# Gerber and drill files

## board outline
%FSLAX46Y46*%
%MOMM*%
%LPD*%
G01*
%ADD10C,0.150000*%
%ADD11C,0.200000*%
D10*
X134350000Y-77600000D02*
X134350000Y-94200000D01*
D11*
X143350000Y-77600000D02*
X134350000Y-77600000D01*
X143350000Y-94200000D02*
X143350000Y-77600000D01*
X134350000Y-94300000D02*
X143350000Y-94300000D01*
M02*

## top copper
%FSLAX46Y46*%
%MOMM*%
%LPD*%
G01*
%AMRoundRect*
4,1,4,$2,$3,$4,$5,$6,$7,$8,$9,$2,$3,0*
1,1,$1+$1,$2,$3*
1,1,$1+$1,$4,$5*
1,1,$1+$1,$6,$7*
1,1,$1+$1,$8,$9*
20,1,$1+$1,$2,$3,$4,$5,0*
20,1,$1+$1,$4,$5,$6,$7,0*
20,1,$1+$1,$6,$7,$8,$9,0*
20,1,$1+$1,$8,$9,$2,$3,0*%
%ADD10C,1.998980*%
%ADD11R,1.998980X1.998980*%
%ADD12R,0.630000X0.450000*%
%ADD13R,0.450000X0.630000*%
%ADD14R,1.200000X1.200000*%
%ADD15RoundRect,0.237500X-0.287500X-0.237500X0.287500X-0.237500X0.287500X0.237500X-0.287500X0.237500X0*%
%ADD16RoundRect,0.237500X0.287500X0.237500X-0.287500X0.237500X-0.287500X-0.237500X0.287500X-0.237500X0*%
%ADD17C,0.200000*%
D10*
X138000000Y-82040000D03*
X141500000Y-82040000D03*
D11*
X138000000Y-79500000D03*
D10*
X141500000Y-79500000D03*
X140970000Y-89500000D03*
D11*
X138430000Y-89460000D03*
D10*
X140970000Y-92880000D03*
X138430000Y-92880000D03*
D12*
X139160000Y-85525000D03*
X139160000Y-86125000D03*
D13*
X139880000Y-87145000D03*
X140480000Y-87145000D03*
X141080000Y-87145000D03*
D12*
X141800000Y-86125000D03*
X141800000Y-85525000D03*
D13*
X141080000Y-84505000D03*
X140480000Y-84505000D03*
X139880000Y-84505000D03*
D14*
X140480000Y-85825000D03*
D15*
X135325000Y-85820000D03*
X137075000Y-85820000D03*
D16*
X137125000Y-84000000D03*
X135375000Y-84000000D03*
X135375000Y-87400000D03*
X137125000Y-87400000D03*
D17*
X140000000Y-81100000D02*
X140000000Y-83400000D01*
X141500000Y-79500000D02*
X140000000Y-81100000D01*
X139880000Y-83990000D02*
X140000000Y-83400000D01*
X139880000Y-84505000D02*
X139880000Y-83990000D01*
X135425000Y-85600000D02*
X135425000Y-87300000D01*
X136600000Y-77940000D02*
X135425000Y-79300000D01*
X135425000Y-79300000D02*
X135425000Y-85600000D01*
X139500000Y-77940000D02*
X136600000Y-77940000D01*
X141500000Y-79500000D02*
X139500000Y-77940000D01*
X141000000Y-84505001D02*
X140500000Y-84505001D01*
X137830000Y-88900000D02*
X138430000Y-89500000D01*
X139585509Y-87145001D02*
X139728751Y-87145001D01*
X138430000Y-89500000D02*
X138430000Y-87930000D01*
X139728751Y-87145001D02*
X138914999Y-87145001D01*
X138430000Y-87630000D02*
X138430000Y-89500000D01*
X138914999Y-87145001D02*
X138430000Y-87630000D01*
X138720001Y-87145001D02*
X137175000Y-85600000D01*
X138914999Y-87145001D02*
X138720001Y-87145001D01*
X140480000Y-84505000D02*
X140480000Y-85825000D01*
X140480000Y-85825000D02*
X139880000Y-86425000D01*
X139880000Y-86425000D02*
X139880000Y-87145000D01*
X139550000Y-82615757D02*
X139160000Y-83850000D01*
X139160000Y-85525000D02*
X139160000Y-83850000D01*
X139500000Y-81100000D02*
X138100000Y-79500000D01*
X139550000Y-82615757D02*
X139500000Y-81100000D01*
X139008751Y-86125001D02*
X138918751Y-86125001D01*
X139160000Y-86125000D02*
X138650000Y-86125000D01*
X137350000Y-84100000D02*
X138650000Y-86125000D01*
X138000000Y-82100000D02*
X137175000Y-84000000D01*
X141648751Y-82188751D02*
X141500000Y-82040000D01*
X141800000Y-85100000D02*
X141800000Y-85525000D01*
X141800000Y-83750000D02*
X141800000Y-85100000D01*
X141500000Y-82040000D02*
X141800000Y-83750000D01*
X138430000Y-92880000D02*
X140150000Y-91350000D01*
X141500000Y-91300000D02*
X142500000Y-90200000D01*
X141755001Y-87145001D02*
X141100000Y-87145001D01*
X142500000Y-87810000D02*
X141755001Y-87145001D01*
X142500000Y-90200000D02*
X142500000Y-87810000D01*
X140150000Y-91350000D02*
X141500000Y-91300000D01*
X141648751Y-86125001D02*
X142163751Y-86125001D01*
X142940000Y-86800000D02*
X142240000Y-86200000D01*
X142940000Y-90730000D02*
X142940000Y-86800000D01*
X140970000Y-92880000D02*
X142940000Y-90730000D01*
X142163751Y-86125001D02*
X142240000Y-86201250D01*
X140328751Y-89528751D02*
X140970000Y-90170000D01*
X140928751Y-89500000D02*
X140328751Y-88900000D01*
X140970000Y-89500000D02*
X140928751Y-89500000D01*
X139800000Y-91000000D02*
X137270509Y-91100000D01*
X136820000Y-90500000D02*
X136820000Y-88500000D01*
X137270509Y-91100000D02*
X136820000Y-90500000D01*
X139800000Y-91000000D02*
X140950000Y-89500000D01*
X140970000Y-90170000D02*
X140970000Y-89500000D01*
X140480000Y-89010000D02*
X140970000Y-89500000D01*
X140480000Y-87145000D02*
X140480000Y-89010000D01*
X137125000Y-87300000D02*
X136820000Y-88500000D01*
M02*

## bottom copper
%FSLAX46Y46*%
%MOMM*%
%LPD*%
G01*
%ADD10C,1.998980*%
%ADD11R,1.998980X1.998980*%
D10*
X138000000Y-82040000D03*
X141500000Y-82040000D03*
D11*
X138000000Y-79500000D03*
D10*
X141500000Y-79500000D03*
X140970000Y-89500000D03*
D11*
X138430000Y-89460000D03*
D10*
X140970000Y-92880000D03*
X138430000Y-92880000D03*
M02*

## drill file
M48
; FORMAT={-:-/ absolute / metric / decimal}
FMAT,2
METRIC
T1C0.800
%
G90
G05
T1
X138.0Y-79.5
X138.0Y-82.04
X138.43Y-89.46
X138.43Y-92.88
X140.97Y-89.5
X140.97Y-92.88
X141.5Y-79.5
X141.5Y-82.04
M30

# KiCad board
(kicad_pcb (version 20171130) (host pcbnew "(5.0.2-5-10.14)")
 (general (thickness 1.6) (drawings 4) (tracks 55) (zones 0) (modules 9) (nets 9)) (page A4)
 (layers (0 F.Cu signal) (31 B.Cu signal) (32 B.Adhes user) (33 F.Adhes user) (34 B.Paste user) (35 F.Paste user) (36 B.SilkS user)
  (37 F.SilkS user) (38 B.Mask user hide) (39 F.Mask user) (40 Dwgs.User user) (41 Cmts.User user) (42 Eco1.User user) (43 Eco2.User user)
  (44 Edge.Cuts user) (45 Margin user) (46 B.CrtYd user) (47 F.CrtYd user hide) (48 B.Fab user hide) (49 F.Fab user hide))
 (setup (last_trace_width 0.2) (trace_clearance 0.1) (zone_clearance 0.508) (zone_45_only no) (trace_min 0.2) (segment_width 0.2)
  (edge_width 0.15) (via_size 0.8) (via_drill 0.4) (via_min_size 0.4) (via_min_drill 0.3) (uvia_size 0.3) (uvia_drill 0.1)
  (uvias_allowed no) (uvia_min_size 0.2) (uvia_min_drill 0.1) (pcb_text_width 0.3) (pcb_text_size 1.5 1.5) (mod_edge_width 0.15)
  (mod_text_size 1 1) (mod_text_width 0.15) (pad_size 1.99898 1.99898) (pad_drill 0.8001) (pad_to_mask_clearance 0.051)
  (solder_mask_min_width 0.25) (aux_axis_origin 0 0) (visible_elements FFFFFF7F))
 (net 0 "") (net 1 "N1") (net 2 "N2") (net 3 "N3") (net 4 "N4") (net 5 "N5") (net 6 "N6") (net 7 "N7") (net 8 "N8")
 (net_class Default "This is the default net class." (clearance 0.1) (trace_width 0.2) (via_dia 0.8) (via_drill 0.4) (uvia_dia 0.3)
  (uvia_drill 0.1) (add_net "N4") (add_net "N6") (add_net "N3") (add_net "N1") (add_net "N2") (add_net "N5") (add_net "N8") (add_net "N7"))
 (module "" (layer F.Cu) (at 140.97 77.47)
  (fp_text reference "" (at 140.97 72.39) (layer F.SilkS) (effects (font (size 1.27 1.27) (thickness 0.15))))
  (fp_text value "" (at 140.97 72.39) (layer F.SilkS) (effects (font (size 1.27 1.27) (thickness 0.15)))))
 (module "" (layer F.Cu) (at 140.97 77.47)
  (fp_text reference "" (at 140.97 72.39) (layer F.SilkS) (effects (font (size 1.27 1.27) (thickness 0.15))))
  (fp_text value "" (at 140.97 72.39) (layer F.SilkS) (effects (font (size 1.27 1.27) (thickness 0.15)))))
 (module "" (layer F.Cu) (at 140.97 72.39)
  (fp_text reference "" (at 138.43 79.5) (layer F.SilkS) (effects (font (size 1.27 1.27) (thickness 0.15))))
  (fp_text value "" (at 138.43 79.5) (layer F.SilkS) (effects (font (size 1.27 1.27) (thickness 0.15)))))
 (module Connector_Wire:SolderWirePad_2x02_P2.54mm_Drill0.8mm (layer F.Cu) (at 138.43 79.5)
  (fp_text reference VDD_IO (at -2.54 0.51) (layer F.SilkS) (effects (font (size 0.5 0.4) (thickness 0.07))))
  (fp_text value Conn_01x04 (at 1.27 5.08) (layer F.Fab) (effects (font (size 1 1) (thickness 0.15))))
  (pad 3 thru_hole circle (at -0.43 2.54) (size 1.99898 1.99898) (drill 0.8001) (layers *.Cu *.Mask) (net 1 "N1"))
  (pad 4 thru_hole circle (at 3.07 2.54) (size 1.99898 1.99898) (drill 0.8001) (layers *.Cu *.Mask) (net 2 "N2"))
  (pad 1 thru_hole rect (at -0.43 0) (size 1.99898 1.99898) (drill 0.8001) (layers *.Cu *.Mask) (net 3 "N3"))
  (pad 2 thru_hole circle (at 3.07 0) (size 1.99898 1.99898) (drill 0.8001) (layers *.Cu *.Mask) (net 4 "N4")))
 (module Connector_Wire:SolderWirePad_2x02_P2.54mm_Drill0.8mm (layer F.Cu) (at 138.43 89.5)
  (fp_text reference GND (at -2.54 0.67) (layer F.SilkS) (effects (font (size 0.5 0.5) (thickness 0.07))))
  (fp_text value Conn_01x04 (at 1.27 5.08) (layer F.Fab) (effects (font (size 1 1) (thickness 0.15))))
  (pad 2 thru_hole circle (at 2.54 0) (size 1.99898 1.99898) (drill 0.8001) (layers *.Cu *.Mask) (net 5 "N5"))
  (pad 1 thru_hole rect (at 0 -0.04) (size 1.99898 1.99898) (drill 0.8001) (layers *.Cu *.Mask) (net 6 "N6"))
  (pad 4 thru_hole circle (at 2.54 3.38) (size 1.99898 1.99898) (drill 0.8001) (layers *.Cu *.Mask) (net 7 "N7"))
  (pad 3 thru_hole circle (at 0 3.38) (size 1.99898 1.99898) (drill 0.8001) (layers *.Cu *.Mask) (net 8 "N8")))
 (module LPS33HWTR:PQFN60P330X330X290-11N (layer F.Cu) (at 140.48 85.825)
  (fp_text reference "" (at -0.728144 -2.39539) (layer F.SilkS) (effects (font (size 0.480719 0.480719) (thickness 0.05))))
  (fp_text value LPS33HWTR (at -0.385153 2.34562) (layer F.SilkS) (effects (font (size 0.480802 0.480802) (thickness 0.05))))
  (pad 1 smd rect (at -1.32 -0.3) (size 0.63 0.45) (layers F.Cu F.Paste F.Mask) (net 3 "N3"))
  (pad 2 smd rect (at -1.32 0.3) (size 0.63 0.45) (layers F.Cu F.Paste F.Mask) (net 1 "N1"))
  (pad 3 smd rect (at -0.6 1.32 90) (size 0.63 0.45) (layers F.Cu F.Paste F.Mask) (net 6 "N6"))
  (pad 4 smd rect (at 0 1.32 90) (size 0.63 0.45) (layers F.Cu F.Paste F.Mask) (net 5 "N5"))
  (pad 5 smd rect (at 0.6 1.32 90) (size 0.63 0.45) (layers F.Cu F.Paste F.Mask) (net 8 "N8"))
  (pad 6 smd rect (at 1.32 0.3 180) (size 0.63 0.45) (layers F.Cu F.Paste F.Mask) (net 7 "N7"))
  (pad 7 smd rect (at 1.32 -0.3 180) (size 0.63 0.45) (layers F.Cu F.Paste F.Mask) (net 2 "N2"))
  (pad 8 smd rect (at 0.6 -1.32 270) (size 0.63 0.45) (layers F.Cu F.Paste F.Mask) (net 6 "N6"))
  (pad 9 smd rect (at 0 -1.32 270) (size 0.63 0.45) (layers F.Cu F.Paste F.Mask) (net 6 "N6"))
  (pad 10 smd rect (at -0.6 -1.32 270) (size 0.63 0.45) (layers F.Cu F.Paste F.Mask) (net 4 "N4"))
  (pad EP smd rect (at 0 0) (size 1.2 1.2) (layers F.Cu F.Paste F.Mask) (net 6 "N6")))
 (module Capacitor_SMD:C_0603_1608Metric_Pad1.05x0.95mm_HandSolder (layer F.Cu) (at 136.2 85.82)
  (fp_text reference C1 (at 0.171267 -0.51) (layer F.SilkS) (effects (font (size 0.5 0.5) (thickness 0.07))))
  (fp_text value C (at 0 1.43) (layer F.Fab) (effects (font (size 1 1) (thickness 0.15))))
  (pad 1 smd roundrect (at -0.875 0) (size 1.05 0.95) (layers F.Cu F.Paste F.Mask) (roundrect_rratio 0.25) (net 4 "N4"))
  (pad 2 smd roundrect (at 0.875 0) (size 1.05 0.95) (layers F.Cu F.Paste F.Mask) (roundrect_rratio 0.25) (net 6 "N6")))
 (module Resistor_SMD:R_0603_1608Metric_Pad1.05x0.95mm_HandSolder (layer F.Cu) (at 136.25 84 180)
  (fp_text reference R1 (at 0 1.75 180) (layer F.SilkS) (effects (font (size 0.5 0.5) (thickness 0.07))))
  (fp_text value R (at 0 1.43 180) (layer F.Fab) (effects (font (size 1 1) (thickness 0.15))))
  (pad 1 smd roundrect (at -0.875 0 180) (size 1.05 0.95) (layers F.Cu F.Paste F.Mask) (roundrect_rratio 0.25) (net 1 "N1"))
  (pad 2 smd roundrect (at 0.875 0 180) (size 1.05 0.95) (layers F.Cu F.Paste F.Mask) (roundrect_rratio 0.25) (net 4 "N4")))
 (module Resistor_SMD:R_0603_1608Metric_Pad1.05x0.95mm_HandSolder (layer F.Cu) (at 136.25 87.4 180)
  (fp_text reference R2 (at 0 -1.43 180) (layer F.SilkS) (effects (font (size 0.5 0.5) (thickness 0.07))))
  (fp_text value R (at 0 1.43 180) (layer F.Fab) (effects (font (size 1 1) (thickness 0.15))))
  (pad 2 smd roundrect (at 0.875 0 180) (size 1.05 0.95) (layers F.Cu F.Paste F.Mask) (roundrect_rratio 0.25) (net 4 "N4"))
  (pad 1 smd roundrect (at -0.875 0 180) (size 1.05 0.95) (layers F.Cu F.Paste F.Mask) (roundrect_rratio 0.25) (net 5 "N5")))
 (gr_line (start 134.35 77.6) (end 134.35 94.2) (layer Edge.Cuts) (width 0.15))
 (gr_line (start 143.35 77.6) (end 134.35 77.6) (layer Edge.Cuts) (width 0.2))
 (gr_line (start 143.35 94.2) (end 143.35 77.6) (layer Edge.Cuts) (width 0.2))
 (gr_line (start 134.35 94.3) (end 143.35 94.3) (layer Edge.Cuts) (width 0.2))
 (segment (start 140 81.1) (end 140 83.4) (width 0.2) (layer F.Cu) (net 4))
 (segment (start 141.5 79.5) (end 140 81.1) (width 0.2) (layer F.Cu) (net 4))
 (segment (start 139.88 83.99) (end 140 83.4) (width 0.2) (layer F.Cu) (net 4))
 (segment (start 139.88 84.505) (end 139.88 83.99) (width 0.2) (layer F.Cu) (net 4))
 (segment (start 135.425 85.6) (end 135.425 87.3) (width 0.2) (layer F.Cu) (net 4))
 (segment (start 136.6 77.94) (end 135.425 79.3) (width 0.2) (layer F.Cu) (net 4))
 (segment (start 135.425 79.3) (end 135.425 85.6) (width 0.2) (layer F.Cu) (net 4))
 (segment (start 139.5 77.94) (end 136.6 77.94) (width 0.2) (layer F.Cu) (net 4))
 (segment (start 141.5 79.5) (end 139.5 77.94) (width 0.2) (layer F.Cu) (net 4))
 (segment (start 141 84.505001) (end 140.5 84.505001) (width 0.2) (layer F.Cu) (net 6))
 (segment (start 137.83 88.9) (end 138.43 89.5) (width 0.2) (layer F.Cu) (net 6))
 (segment (start 139.585509 87.145001) (end 139.728751 87.145001) (width 0.2) (layer F.Cu) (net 6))
 (segment (start 138.43 89.5) (end 138.43 87.93) (width 0.2) (layer F.Cu) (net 6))
 (segment (start 139.728751 87.145001) (end 138.914999 87.145001) (width 0.2) (layer F.Cu) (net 6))
 (segment (start 138.43 87.63) (end 138.43 89.5) (width 0.2) (layer F.Cu) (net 6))
 (segment (start 138.914999 87.145001) (end 138.43 87.63) (width 0.2) (layer F.Cu) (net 6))
 (segment (start 138.720001 87.145001) (end 137.175 85.6) (width 0.2) (layer F.Cu) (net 6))
 (segment (start 138.914999 87.145001) (end 138.720001 87.145001) (width 0.2) (layer F.Cu) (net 6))
 (segment (start 140.48 84.505) (end 140.48 85.825) (width 0.2) (layer F.Cu) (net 6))
 (segment (start 140.48 85.825) (end 139.88 86.425) (width 0.2) (layer F.Cu) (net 6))
 (segment (start 139.88 86.425) (end 139.88 87.145) (width 0.2) (layer F.Cu) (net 6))
 (segment (start 139.55 82.615757) (end 139.16 83.85) (width 0.2) (layer F.Cu) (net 3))
 (segment (start 139.16 85.525) (end 139.16 83.85) (width 0.2) (layer F.Cu) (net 3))
 (segment (start 139.5 81.1) (end 138.1 79.5) (width 0.2) (layer F.Cu) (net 3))
 (segment (start 139.55 82.615757) (end 139.5 81.1) (width 0.2) (layer F.Cu) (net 3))
 (segment (start 139.008751 86.125001) (end 138.918751 86.125001) (width 0.2) (layer F.Cu) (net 1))
 (segment (start 139.16 86.125) (end 138.65 86.125) (width 0.2) (layer F.Cu) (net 1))
 (segment (start 137.35 84.1) (end 138.65 86.125) (width 0.2) (layer F.Cu) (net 1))
 (segment (start 138 82.1) (end 137.175 84) (width 0.2) (layer F.Cu) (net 1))
 (segment (start 141.648751 82.188751) (end 141.5 82.04) (width 0.2) (layer F.Cu) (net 2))
 (segment (start 141.8 85.1) (end 141.8 85.525) (width 0.2) (layer F.Cu) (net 2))
 (segment (start 141.8 83.75) (end 141.8 85.1) (width 0.2) (layer F.Cu) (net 2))
 (segment (start 141.5 82.04) (end 141.8 83.75) (width 0.2) (layer F.Cu) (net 2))
 (segment (start 138.43 92.88) (end 140.15 91.35) (width 0.2) (layer F.Cu) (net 8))
 (segment (start 141.5 91.3) (end 142.5 90.2) (width 0.2) (layer F.Cu) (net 8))
 (segment (start 141.755001 87.145001) (end 141.1 87.145001) (width 0.2) (layer F.Cu) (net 8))
 (segment (start 142.5 87.81) (end 141.755001 87.145001) (width 0.2) (layer F.Cu) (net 8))
 (segment (start 142.5 90.2) (end 142.5 87.81) (width 0.2) (layer F.Cu) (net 8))
 (segment (start 140.15 91.35) (end 141.5 91.3) (width 0.2) (layer F.Cu) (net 8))
 (segment (start 141.648751 86.125001) (end 142.163751 86.125001) (width 0.2) (layer F.Cu) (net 7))
 (segment (start 142.94 86.8) (end 142.24 86.2) (width 0.2) (layer F.Cu) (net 7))
 (segment (start 142.94 90.73) (end 142.94 86.8) (width 0.2) (layer F.Cu) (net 7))
 (segment (start 140.97 92.88) (end 142.94 90.73) (width 0.2) (layer F.Cu) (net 7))
 (segment (start 142.163751 86.125001) (end 142.24 86.20125) (width 0.2) (layer F.Cu) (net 7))
 (segment (start 140.328751 89.528751) (end 140.97 90.17) (width 0.2) (layer F.Cu) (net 5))
 (segment (start 140.928751 89.5) (end 140.328751 88.9) (width 0.2) (layer F.Cu) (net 5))
 (segment (start 140.97 89.5) (end 140.928751 89.5) (width 0.2) (layer F.Cu) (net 5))
 (segment (start 139.8 91) (end 137.270509 91.1) (width 0.2) (layer F.Cu) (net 5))
 (segment (start 136.82 90.5) (end 136.82 88.5) (width 0.2) (layer F.Cu) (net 5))
 (segment (start 137.270509 91.1) (end 136.82 90.5) (width 0.2) (layer F.Cu) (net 5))
 (segment (start 139.8 91) (end 140.95 89.5) (width 0.2) (layer F.Cu) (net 5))
 (segment (start 140.97 90.17) (end 140.97 89.5) (width 0.2) (layer F.Cu) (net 5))
 (segment (start 140.48 89.01) (end 140.97 89.5) (width 0.2) (layer F.Cu) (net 5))
 (segment (start 140.48 87.145) (end 140.48 89.01) (width 0.2) (layer F.Cu) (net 5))
 (segment (start 137.125 87.3) (end 136.82 88.5) (width 0.2) (layer F.Cu) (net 5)))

